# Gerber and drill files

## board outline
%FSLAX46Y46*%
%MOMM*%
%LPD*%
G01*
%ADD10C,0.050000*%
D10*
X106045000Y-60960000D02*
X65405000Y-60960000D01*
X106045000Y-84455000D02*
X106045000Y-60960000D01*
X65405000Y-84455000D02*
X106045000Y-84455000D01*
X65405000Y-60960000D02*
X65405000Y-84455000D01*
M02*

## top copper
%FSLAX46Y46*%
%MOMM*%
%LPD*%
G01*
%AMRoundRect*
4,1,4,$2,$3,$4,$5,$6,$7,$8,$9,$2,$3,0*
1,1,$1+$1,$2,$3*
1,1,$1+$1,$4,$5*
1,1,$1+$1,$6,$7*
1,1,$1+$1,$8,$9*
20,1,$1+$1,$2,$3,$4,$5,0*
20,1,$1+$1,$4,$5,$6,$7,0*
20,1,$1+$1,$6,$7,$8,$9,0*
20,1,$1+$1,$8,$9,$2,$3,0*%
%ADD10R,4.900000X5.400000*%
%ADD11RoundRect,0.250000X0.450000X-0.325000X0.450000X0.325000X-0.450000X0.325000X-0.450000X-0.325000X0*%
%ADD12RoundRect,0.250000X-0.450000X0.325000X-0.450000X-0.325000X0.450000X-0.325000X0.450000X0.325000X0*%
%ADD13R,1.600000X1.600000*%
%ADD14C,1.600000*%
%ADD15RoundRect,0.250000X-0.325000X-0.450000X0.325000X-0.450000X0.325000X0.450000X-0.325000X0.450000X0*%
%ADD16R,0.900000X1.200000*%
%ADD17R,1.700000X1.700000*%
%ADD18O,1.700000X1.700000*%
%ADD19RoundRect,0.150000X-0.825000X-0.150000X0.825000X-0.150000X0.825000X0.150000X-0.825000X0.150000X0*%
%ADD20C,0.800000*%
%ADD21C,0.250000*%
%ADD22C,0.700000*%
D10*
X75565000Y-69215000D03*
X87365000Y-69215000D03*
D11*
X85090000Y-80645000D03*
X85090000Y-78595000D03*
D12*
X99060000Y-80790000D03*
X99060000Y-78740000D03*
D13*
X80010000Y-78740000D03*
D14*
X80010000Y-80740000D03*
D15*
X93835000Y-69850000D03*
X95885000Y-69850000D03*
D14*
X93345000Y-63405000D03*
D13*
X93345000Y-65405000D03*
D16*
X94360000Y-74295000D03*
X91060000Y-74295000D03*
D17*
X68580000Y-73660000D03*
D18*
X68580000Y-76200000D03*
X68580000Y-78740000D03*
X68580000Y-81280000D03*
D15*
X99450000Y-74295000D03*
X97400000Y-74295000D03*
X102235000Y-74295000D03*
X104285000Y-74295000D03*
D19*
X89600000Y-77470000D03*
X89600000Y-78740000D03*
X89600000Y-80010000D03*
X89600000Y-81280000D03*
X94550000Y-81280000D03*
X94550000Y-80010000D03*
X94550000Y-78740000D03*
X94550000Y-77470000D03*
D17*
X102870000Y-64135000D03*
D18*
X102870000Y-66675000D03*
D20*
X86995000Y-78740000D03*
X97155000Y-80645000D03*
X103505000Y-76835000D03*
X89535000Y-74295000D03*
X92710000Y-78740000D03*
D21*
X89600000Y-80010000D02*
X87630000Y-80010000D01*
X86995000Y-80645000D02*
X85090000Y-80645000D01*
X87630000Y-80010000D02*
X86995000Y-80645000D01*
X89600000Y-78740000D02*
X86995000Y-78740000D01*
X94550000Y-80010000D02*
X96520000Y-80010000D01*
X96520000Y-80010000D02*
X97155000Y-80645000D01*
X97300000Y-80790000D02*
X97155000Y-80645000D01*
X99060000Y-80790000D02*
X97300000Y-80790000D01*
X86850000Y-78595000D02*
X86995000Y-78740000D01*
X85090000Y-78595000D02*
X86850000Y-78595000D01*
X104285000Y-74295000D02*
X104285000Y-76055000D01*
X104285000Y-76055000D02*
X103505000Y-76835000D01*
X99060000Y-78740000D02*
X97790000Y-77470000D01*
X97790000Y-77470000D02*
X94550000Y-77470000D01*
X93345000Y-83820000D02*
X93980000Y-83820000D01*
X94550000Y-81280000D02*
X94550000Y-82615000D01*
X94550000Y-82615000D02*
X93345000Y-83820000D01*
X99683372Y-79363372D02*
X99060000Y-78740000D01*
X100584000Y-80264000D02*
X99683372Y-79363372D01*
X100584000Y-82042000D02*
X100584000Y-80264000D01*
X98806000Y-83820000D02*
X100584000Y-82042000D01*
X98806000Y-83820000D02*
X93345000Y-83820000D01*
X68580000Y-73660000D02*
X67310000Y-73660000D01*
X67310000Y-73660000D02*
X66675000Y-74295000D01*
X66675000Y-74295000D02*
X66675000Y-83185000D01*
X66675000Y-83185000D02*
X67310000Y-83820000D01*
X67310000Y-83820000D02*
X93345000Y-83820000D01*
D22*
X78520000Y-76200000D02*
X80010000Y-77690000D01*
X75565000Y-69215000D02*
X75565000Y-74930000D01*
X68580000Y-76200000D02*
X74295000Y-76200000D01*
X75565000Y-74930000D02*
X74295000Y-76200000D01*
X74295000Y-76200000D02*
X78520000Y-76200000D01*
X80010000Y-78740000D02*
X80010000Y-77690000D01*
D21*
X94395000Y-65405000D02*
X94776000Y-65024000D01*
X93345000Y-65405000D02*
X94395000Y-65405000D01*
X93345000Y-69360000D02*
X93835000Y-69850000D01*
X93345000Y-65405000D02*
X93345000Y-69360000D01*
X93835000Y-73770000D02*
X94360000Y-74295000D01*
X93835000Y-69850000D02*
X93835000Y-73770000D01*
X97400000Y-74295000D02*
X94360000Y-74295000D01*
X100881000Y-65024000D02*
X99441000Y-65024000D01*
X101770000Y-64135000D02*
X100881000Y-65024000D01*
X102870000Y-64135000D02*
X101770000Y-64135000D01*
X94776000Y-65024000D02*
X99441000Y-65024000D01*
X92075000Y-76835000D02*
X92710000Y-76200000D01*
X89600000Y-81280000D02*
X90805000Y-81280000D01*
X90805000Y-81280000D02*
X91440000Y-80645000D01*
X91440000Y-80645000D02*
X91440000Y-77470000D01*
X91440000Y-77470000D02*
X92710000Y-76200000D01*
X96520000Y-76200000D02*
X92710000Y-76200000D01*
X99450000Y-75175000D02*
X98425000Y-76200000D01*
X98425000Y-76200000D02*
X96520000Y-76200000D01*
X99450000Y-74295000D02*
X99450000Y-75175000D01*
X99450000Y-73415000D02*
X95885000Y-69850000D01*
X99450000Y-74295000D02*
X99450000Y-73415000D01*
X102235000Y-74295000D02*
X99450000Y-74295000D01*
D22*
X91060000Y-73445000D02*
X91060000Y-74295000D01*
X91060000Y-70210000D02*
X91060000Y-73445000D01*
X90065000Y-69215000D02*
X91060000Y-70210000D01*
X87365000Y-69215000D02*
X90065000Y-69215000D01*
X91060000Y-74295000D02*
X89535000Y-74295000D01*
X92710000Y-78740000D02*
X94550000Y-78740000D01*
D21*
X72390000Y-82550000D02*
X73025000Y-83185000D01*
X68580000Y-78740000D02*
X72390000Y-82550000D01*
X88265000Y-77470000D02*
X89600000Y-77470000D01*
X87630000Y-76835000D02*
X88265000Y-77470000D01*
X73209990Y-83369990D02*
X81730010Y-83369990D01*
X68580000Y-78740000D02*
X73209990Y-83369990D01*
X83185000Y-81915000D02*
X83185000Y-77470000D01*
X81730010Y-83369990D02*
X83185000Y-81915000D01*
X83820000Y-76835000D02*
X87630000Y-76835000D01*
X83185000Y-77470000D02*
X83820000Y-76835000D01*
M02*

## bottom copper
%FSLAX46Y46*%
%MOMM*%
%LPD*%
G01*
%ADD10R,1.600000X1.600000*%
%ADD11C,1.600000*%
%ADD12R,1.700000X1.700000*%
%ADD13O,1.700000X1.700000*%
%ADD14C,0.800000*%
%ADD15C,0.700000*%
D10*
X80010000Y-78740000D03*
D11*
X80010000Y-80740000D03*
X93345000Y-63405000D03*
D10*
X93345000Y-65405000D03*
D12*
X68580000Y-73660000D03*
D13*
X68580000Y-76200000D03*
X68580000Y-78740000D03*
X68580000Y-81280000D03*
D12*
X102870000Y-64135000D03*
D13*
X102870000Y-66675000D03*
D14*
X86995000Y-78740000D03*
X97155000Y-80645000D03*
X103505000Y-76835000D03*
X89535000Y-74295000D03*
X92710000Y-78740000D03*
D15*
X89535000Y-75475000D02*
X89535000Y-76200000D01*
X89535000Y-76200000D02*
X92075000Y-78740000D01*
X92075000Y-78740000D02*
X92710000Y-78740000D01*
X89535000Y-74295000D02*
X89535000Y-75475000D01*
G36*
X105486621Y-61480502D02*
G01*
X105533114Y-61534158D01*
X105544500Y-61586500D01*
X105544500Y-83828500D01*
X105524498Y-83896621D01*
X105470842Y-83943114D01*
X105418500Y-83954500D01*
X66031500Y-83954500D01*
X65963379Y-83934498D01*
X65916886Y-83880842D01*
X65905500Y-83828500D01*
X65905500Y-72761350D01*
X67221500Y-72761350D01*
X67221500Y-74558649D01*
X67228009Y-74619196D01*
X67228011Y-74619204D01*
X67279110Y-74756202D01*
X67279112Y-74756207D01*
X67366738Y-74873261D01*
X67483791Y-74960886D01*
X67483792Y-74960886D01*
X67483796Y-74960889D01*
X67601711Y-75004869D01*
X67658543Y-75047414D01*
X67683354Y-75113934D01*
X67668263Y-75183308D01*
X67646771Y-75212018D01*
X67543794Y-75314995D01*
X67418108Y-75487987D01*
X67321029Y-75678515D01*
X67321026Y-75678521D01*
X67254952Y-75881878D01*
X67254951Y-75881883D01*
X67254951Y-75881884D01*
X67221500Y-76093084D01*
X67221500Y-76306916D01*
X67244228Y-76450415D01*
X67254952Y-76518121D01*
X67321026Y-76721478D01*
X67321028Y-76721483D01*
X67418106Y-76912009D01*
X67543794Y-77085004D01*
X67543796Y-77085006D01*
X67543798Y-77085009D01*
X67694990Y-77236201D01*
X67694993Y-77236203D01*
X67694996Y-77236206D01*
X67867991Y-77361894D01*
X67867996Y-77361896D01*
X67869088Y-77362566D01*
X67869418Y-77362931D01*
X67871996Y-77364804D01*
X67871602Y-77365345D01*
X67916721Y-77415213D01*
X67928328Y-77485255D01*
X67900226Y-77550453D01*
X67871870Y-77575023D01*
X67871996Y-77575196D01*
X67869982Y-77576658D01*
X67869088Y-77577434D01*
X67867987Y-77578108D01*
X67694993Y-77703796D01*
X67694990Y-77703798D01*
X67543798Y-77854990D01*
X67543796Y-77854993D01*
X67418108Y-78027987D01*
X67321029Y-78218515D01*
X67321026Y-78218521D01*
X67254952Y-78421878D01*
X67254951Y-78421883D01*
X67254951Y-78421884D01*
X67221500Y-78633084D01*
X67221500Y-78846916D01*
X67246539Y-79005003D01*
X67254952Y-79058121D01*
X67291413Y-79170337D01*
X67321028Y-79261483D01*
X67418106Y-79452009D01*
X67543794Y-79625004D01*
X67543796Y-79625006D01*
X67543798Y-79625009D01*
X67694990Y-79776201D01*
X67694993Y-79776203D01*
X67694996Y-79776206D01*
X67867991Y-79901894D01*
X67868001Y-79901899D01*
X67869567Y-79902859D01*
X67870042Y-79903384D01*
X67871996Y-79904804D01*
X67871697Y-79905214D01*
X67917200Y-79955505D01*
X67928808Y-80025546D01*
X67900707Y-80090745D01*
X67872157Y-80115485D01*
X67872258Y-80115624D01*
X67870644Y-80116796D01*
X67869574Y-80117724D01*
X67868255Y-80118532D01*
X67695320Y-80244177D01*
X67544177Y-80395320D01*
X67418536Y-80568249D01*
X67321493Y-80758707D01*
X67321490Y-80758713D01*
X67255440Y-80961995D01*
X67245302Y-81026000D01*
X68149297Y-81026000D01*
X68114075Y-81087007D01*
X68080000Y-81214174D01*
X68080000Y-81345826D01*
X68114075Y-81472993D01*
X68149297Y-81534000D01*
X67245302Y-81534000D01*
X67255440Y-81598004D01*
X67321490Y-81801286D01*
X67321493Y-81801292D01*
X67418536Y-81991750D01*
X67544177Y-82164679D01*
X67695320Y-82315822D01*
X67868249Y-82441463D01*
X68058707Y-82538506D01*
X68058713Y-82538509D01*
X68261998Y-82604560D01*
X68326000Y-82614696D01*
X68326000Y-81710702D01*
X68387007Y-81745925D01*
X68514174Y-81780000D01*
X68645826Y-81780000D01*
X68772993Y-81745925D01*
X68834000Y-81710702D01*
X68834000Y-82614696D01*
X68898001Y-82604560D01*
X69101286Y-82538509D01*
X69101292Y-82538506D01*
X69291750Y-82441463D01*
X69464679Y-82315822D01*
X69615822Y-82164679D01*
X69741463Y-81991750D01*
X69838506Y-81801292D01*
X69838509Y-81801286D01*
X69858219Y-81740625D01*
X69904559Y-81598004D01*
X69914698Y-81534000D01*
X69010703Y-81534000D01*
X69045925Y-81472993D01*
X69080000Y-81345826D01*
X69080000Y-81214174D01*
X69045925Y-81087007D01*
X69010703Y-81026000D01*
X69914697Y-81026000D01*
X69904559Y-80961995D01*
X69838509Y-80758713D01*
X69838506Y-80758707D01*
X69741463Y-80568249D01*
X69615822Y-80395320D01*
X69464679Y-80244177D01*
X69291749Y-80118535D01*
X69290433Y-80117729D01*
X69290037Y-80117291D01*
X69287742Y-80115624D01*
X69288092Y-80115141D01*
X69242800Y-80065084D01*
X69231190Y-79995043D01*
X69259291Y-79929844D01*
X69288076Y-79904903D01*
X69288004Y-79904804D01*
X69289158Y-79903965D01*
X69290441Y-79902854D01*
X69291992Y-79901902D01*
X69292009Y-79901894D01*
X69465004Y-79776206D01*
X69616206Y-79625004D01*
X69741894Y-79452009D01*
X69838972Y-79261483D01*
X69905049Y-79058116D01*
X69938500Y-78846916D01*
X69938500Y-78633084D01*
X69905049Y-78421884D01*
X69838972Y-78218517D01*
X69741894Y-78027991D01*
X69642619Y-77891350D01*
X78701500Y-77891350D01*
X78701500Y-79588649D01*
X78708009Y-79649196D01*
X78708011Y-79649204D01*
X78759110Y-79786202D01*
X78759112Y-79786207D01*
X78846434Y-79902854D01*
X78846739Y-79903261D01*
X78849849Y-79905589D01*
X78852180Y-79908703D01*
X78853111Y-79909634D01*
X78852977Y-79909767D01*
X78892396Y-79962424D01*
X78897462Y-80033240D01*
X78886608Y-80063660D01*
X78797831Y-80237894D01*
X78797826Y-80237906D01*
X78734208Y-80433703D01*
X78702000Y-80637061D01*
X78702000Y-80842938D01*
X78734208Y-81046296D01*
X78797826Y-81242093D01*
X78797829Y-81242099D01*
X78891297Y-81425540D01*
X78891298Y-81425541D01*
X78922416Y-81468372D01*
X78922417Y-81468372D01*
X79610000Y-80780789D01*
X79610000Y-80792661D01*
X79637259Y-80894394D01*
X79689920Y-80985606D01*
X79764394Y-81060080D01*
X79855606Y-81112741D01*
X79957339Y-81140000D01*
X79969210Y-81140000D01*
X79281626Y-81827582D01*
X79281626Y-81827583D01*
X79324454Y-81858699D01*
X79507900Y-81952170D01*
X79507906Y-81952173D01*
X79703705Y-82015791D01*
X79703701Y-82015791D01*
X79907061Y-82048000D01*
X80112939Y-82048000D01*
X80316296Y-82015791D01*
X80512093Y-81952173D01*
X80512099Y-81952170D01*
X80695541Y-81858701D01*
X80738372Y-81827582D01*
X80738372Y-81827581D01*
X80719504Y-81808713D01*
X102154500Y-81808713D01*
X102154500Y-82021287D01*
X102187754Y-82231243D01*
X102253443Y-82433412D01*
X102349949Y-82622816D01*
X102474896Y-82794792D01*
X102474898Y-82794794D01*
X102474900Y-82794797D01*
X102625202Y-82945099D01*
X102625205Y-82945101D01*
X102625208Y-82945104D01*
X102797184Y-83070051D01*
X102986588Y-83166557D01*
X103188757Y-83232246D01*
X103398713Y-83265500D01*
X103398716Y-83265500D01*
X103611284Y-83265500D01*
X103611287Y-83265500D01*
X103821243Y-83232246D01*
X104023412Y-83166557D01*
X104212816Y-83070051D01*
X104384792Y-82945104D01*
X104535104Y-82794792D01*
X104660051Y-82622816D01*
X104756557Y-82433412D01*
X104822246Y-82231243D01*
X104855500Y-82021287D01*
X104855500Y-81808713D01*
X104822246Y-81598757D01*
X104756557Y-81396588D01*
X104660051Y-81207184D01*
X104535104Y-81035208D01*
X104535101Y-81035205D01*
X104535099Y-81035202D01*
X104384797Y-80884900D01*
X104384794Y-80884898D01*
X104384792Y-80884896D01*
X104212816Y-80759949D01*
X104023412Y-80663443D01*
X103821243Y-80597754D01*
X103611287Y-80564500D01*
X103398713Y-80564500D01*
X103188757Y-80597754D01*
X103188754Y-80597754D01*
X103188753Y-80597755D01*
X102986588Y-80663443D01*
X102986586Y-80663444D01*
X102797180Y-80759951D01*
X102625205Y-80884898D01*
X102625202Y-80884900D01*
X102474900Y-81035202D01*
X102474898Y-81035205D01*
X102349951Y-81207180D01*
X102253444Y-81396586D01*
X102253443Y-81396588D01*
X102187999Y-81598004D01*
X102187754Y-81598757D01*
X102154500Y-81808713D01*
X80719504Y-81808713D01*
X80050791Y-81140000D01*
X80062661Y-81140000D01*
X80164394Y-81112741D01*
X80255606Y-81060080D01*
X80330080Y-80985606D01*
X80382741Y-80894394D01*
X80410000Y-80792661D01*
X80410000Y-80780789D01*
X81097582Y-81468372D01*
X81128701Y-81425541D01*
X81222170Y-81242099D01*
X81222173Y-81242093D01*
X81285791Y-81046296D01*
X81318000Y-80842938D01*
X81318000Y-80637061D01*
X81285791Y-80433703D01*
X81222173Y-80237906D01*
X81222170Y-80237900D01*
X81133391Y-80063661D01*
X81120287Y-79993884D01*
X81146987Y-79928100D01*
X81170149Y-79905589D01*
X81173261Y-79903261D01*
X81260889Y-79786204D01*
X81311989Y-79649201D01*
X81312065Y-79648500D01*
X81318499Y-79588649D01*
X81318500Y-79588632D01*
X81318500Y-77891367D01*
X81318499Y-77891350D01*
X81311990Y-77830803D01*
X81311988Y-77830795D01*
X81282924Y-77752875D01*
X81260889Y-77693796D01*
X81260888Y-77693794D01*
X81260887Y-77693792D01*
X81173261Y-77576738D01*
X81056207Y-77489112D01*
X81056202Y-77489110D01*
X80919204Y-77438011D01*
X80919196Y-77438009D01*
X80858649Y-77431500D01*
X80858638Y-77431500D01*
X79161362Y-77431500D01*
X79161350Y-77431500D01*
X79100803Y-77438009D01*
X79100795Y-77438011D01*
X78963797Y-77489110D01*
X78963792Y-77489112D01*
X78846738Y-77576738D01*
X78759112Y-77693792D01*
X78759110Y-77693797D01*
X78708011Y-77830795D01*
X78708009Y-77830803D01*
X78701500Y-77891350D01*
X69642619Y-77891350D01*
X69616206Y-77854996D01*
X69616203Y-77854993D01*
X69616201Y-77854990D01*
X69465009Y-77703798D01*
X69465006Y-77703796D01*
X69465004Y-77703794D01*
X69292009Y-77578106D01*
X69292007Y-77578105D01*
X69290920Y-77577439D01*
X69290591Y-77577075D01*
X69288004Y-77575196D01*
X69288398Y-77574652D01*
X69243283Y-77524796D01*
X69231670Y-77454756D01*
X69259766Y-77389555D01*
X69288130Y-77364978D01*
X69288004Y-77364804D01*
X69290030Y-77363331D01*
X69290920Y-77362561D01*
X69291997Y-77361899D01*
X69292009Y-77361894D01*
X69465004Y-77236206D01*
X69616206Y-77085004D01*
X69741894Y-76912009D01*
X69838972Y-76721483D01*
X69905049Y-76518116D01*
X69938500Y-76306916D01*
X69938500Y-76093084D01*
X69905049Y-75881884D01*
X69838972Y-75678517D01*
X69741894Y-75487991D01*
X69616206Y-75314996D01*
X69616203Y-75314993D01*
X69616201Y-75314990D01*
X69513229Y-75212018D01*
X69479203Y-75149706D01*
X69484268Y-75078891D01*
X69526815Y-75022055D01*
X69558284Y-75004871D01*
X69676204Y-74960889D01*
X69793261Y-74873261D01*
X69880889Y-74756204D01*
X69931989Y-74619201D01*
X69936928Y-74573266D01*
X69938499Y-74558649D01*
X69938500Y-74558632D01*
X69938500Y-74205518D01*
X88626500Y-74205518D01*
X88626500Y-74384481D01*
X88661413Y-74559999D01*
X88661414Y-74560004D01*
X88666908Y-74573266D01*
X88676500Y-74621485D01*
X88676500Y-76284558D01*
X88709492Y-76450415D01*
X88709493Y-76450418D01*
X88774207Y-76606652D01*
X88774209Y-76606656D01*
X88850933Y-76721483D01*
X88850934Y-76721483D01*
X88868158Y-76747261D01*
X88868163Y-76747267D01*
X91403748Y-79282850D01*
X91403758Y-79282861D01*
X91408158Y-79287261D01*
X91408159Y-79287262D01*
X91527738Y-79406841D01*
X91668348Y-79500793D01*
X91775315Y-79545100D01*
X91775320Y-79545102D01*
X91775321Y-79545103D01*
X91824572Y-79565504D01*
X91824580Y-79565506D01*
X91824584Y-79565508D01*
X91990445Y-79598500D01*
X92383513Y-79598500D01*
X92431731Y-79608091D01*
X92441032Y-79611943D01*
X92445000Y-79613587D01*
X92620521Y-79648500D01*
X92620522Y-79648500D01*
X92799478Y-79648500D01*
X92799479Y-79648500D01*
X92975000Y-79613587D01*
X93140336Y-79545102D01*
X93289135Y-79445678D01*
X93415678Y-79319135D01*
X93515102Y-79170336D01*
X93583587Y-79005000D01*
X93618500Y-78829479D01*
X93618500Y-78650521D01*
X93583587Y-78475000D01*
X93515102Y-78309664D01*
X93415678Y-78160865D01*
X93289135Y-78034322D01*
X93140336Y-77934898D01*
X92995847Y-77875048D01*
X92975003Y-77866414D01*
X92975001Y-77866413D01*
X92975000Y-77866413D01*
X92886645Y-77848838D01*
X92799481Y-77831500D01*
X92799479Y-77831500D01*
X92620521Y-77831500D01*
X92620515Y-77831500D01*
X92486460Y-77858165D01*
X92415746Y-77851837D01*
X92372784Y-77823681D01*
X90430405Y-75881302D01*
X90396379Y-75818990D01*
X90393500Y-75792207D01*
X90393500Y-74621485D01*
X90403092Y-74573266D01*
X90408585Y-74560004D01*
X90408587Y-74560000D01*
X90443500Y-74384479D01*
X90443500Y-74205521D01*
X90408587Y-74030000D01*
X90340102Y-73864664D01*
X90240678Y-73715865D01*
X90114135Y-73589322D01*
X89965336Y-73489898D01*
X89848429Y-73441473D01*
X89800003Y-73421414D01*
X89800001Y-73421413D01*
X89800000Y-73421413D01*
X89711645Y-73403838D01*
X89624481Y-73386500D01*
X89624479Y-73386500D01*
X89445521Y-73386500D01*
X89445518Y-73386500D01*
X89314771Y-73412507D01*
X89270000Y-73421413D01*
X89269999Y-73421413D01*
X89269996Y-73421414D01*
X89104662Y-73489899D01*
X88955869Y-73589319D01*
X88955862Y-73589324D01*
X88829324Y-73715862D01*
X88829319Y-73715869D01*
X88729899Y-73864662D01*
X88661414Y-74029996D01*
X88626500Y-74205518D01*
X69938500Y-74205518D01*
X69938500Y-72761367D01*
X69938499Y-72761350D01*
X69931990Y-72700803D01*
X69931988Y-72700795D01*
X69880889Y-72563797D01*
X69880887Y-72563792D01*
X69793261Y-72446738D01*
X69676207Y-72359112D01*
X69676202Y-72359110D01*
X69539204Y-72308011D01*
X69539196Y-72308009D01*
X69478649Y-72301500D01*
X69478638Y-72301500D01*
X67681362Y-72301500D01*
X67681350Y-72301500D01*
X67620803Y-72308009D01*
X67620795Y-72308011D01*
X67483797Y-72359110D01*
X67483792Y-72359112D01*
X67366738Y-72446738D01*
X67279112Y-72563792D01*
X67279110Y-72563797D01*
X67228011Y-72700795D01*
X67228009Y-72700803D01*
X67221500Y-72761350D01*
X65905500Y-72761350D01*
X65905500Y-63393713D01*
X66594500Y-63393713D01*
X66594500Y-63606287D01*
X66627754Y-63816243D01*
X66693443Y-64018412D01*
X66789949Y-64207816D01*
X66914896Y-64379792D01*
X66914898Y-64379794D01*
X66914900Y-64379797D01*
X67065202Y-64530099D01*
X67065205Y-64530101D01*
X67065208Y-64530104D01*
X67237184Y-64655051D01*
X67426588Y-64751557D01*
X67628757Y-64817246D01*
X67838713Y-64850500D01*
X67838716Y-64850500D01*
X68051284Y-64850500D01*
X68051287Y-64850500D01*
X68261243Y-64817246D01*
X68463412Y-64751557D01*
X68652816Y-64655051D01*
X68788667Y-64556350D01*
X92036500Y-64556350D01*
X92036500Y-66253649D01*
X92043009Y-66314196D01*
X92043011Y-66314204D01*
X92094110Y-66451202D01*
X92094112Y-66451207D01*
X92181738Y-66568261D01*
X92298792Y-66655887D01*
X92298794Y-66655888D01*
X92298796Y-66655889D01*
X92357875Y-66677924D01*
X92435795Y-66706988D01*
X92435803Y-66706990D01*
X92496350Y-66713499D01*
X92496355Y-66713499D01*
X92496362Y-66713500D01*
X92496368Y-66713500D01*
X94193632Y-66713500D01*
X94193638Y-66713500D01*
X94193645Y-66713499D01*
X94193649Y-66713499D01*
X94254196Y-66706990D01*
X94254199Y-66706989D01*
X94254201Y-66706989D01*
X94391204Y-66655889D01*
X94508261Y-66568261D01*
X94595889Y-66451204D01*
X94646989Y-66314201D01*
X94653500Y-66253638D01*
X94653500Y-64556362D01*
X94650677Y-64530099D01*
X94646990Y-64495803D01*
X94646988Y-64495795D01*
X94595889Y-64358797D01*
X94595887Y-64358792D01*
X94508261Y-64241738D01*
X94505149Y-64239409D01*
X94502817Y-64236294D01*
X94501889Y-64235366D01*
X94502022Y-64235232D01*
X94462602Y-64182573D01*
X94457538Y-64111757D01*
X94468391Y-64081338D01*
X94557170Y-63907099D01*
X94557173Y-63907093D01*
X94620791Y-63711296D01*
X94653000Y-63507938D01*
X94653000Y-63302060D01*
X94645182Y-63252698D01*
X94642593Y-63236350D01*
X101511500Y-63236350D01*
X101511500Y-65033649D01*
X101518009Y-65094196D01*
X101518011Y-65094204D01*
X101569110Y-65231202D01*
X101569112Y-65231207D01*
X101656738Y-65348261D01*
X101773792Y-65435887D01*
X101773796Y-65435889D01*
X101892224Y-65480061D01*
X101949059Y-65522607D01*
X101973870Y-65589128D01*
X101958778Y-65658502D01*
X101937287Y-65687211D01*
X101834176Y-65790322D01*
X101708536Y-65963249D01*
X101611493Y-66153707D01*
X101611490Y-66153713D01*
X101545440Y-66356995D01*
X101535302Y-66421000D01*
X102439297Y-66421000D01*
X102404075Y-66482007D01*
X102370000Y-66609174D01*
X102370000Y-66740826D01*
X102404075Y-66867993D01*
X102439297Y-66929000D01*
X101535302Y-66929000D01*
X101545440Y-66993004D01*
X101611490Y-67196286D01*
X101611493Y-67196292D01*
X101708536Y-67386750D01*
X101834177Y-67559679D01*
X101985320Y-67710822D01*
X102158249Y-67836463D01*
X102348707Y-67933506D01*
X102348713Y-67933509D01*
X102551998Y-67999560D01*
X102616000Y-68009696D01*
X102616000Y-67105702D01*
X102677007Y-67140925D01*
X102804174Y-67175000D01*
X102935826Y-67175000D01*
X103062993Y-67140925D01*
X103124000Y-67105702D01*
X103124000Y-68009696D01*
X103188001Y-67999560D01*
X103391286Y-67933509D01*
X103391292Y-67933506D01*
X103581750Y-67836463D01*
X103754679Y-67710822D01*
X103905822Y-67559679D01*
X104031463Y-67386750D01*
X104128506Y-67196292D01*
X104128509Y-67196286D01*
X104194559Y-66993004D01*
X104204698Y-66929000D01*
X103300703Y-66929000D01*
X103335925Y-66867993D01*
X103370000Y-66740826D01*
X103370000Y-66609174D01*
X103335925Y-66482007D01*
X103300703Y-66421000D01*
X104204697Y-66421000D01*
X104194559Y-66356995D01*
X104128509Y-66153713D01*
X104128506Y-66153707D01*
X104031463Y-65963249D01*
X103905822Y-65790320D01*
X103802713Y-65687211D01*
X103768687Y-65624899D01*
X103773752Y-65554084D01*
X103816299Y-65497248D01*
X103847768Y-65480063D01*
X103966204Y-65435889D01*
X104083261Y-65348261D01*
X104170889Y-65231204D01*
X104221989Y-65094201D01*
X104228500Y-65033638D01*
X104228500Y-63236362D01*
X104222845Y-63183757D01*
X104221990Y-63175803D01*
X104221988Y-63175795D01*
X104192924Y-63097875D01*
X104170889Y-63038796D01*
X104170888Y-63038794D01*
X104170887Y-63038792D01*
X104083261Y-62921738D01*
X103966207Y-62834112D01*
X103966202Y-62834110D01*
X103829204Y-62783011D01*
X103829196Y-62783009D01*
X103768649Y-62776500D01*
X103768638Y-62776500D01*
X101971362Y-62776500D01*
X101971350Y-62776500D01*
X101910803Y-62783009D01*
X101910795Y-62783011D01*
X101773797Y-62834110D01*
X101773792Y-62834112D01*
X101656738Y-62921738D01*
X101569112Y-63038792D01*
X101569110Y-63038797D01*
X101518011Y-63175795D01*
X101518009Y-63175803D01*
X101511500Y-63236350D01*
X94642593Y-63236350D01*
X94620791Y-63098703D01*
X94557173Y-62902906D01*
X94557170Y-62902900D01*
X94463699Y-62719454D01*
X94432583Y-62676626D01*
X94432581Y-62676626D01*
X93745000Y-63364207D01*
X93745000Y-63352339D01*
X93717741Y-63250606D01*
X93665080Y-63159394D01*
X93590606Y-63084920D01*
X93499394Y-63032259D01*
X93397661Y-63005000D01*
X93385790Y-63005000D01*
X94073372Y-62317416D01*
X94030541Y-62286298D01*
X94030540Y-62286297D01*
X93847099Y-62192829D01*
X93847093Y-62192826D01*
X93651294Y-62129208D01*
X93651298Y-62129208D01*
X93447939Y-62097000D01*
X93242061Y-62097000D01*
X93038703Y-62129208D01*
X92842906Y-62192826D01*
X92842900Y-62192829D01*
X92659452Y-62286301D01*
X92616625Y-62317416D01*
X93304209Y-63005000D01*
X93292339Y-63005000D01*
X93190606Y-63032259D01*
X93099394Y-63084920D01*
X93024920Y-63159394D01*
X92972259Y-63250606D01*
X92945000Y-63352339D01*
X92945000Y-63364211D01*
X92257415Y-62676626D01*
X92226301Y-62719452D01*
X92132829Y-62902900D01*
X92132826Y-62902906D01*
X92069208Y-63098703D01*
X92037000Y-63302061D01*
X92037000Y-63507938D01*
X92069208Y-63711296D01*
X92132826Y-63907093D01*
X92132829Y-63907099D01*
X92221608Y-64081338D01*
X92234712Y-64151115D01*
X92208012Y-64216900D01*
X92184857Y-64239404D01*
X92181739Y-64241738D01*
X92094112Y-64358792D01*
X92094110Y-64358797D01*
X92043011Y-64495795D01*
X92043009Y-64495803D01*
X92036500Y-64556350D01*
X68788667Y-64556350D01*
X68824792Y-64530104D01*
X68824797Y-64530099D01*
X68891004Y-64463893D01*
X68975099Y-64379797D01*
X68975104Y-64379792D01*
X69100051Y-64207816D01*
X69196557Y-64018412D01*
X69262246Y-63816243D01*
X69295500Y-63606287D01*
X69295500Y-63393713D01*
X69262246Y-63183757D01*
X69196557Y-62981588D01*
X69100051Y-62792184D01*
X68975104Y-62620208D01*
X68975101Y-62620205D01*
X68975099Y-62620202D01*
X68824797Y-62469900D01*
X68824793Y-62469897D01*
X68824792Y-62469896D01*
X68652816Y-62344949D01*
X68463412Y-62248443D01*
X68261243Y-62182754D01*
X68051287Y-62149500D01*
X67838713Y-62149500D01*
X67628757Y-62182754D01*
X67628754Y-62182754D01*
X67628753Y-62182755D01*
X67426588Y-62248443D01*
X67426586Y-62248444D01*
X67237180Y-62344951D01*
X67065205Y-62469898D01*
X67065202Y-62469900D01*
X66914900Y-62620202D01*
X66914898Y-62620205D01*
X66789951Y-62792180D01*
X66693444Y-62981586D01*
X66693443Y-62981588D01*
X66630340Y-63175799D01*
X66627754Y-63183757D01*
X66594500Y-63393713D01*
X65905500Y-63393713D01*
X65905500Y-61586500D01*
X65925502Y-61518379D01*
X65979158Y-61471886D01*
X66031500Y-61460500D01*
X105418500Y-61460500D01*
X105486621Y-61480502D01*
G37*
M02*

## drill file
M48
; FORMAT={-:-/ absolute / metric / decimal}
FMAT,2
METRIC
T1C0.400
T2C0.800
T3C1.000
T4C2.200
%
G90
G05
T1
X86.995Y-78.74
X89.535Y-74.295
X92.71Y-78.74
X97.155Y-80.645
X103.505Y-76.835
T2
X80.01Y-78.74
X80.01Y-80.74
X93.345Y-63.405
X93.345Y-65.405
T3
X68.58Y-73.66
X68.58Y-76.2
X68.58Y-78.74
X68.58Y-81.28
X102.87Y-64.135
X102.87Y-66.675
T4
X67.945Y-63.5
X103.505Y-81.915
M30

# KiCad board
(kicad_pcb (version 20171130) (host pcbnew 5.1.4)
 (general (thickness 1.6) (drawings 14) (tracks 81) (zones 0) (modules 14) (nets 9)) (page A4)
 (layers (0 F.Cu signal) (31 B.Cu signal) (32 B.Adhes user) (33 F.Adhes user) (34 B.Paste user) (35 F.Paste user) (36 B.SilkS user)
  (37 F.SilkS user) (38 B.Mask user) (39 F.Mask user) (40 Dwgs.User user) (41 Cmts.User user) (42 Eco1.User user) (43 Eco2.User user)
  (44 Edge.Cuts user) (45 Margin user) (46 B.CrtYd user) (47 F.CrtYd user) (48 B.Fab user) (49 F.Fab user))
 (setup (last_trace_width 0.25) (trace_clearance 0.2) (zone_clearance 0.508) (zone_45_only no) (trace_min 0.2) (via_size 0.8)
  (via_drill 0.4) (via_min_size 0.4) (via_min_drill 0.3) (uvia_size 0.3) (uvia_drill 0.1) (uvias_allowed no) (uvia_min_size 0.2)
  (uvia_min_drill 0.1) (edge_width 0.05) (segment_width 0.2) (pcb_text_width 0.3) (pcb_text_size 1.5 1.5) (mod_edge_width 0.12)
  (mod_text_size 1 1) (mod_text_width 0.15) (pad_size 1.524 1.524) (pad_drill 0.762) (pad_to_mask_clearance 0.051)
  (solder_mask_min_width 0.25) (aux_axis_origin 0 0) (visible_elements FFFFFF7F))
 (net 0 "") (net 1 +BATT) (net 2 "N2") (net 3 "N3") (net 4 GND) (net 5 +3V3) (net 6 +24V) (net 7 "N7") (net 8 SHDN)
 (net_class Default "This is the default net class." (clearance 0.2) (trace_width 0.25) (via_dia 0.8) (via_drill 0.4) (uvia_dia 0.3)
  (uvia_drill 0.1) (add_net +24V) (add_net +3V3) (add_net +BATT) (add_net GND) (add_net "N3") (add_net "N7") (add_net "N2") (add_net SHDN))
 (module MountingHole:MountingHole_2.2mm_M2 (layer F.Cu) (at 103.505 81.915)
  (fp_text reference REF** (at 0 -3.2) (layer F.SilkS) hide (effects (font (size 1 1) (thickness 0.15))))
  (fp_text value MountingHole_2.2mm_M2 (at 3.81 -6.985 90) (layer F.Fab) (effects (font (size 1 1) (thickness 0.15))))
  (pad 1 np_thru_hole circle (at 0 0) (size 2.2 2.2) (drill 2.2) (layers *.Cu *.Mask)))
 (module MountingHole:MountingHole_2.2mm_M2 (layer F.Cu) (at 67.945 63.5)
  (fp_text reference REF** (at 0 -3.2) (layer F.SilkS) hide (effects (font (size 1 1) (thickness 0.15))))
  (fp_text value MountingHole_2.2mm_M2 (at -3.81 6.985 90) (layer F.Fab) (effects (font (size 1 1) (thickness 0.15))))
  (pad 1 np_thru_hole circle (at 0 0) (size 2.2 2.2) (drill 2.2) (layers *.Cu *.Mask)))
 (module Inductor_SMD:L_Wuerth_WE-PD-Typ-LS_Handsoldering (layer F.Cu) (at 81.465 69.215)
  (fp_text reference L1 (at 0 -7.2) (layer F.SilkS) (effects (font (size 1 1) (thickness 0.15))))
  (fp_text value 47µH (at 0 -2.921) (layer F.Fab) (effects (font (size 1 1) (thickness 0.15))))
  (pad 1 smd rect (at -5.9 0) (size 4.9 5.4) (layers F.Cu F.Paste F.Mask) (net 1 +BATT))
  (pad 2 smd rect (at 5.9 0) (size 4.9 5.4) (layers F.Cu F.Paste F.Mask) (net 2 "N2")))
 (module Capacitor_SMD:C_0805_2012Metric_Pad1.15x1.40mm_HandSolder (layer F.Cu) (at 85.09 79.62 90)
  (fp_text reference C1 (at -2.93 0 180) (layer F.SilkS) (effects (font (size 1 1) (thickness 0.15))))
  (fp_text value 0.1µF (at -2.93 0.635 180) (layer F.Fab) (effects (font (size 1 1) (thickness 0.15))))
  (pad 1 smd roundrect (at -1.025 0 90) (size 1.15 1.4) (layers F.Cu F.Paste F.Mask) (roundrect_rratio 0.217391) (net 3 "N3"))
  (pad 2 smd roundrect (at 1.025 0 90) (size 1.15 1.4) (layers F.Cu F.Paste F.Mask) (roundrect_rratio 0.217391) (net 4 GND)))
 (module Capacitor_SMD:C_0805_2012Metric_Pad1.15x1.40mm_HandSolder (layer F.Cu) (at 99.06 79.765 270)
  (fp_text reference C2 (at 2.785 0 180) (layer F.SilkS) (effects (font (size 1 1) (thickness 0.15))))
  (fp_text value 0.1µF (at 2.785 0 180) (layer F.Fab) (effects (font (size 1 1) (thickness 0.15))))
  (pad 2 smd roundrect (at 1.025 0 270) (size 1.15 1.4) (layers F.Cu F.Paste F.Mask) (roundrect_rratio 0.217391) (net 4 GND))
  (pad 1 smd roundrect (at -1.025 0 270) (size 1.15 1.4) (layers F.Cu F.Paste F.Mask) (roundrect_rratio 0.217391) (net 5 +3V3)))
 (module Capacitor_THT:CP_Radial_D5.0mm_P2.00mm (layer F.Cu) (at 80.01 78.74 270)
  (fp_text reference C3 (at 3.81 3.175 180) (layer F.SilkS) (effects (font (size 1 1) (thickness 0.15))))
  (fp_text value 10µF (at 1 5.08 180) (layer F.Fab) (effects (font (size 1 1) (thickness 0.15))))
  (pad 1 thru_hole rect (at 0 0 270) (size 1.6 1.6) (drill 0.8) (layers *.Cu *.Mask) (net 1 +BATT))
  (pad 2 thru_hole circle (at 2 0 270) (size 1.6 1.6) (drill 0.8) (layers *.Cu *.Mask) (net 4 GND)))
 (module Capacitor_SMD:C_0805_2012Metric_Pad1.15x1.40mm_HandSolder (layer F.Cu) (at 94.86 69.85)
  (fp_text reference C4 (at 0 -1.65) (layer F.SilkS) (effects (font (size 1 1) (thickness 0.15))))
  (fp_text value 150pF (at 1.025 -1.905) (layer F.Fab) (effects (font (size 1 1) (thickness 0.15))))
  (pad 1 smd roundrect (at -1.025 0) (size 1.15 1.4) (layers F.Cu F.Paste F.Mask) (roundrect_rratio 0.217391) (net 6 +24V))
  (pad 2 smd roundrect (at 1.025 0) (size 1.15 1.4) (layers F.Cu F.Paste F.Mask) (roundrect_rratio 0.217391) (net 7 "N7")))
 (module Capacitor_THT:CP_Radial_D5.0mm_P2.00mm (layer F.Cu) (at 93.345 65.405 90)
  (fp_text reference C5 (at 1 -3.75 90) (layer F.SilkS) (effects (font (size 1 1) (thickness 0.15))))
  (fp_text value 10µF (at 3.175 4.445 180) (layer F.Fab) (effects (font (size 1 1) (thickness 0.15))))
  (pad 2 thru_hole circle (at 2 0 90) (size 1.6 1.6) (drill 0.8) (layers *.Cu *.Mask) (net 4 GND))
  (pad 1 thru_hole rect (at 0 0 90) (size 1.6 1.6) (drill 0.8) (layers *.Cu *.Mask) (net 6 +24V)))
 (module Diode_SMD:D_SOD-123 (layer F.Cu) (at 92.71 74.295 180)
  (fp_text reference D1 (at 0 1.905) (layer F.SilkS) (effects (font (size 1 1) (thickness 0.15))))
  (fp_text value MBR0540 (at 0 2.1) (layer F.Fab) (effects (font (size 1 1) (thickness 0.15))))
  (pad 1 smd rect (at -1.65 0 180) (size 0.9 1.2) (layers F.Cu F.Paste F.Mask) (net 6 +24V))
  (pad 2 smd rect (at 1.65 0 180) (size 0.9 1.2) (layers F.Cu F.Paste F.Mask) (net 2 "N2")))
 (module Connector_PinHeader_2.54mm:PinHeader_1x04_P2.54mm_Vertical (layer F.Cu) (at 68.58 73.66)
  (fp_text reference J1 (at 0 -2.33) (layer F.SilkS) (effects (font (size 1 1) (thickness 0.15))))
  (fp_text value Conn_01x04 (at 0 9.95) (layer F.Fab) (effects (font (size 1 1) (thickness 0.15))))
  (pad 1 thru_hole rect (at 0 0) (size 1.7 1.7) (drill 1) (layers *.Cu *.Mask) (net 5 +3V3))
  (pad 2 thru_hole oval (at 0 2.54) (size 1.7 1.7) (drill 1) (layers *.Cu *.Mask) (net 1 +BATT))
  (pad 3 thru_hole oval (at 0 5.08) (size 1.7 1.7) (drill 1) (layers *.Cu *.Mask) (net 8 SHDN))
  (pad 4 thru_hole oval (at 0 7.62) (size 1.7 1.7) (drill 1) (layers *.Cu *.Mask) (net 4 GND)))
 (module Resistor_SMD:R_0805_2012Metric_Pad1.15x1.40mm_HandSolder (layer F.Cu) (at 98.425 74.295)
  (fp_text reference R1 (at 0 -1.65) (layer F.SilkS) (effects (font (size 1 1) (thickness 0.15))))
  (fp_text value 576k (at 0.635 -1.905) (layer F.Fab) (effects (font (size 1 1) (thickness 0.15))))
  (pad 2 smd roundrect (at 1.025 0) (size 1.15 1.4) (layers F.Cu F.Paste F.Mask) (roundrect_rratio 0.217391) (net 7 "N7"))
  (pad 1 smd roundrect (at -1.025 0) (size 1.15 1.4) (layers F.Cu F.Paste F.Mask) (roundrect_rratio 0.217391) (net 6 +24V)))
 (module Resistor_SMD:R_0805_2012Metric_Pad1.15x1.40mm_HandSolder (layer F.Cu) (at 103.26 74.295)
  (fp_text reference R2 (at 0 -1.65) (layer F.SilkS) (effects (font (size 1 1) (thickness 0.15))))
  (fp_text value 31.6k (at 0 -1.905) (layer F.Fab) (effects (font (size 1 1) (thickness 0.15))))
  (pad 1 smd roundrect (at -1.025 0) (size 1.15 1.4) (layers F.Cu F.Paste F.Mask) (roundrect_rratio 0.217391) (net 7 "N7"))
  (pad 2 smd roundrect (at 1.025 0) (size 1.15 1.4) (layers F.Cu F.Paste F.Mask) (roundrect_rratio 0.217391) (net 4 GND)))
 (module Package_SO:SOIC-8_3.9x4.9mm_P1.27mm (layer F.Cu) (at 92.075 79.375)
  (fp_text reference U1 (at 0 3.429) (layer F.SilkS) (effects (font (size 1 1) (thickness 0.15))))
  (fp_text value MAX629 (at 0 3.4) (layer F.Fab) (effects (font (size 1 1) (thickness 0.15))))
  (pad 1 smd roundrect (at -2.475 -1.905) (size 1.95 0.6) (layers F.Cu F.Paste F.Mask) (roundrect_rratio 0.25) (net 8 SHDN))
  (pad 2 smd roundrect (at -2.475 -0.635) (size 1.95 0.6) (layers F.Cu F.Paste F.Mask) (roundrect_rratio 0.25) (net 4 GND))
  (pad 3 smd roundrect (at -2.475 0.635) (size 1.95 0.6) (layers F.Cu F.Paste F.Mask) (roundrect_rratio 0.25) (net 3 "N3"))
  (pad 4 smd roundrect (at -2.475 1.905) (size 1.95 0.6) (layers F.Cu F.Paste F.Mask) (roundrect_rratio 0.25) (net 7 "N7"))
  (pad 5 smd roundrect (at 2.475 1.905) (size 1.95 0.6) (layers F.Cu F.Paste F.Mask) (roundrect_rratio 0.25) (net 5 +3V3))
  (pad 6 smd roundrect (at 2.475 0.635) (size 1.95 0.6) (layers F.Cu F.Paste F.Mask) (roundrect_rratio 0.25) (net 4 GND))
  (pad 7 smd roundrect (at 2.475 -0.635) (size 1.95 0.6) (layers F.Cu F.Paste F.Mask) (roundrect_rratio 0.25) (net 2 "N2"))
  (pad 8 smd roundrect (at 2.475 -1.905) (size 1.95 0.6) (layers F.Cu F.Paste F.Mask) (roundrect_rratio 0.25) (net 5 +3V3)))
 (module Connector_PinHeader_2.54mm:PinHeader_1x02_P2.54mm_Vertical (layer F.Cu) (at 102.87 64.135)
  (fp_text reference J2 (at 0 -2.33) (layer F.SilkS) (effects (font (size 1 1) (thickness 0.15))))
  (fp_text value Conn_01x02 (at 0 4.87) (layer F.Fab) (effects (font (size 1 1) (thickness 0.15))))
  (pad 1 thru_hole rect (at 0 0) (size 1.7 1.7) (drill 1) (layers *.Cu *.Mask) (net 6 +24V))
  (pad 2 thru_hole oval (at 0 2.54) (size 1.7 1.7) (drill 1) (layers *.Cu *.Mask) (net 4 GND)))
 (gr_line (start 106.045 60.96) (end 65.405 60.96) (layer Edge.Cuts) (width 0.05))
 (gr_line (start 106.045 84.455) (end 106.045 60.96) (layer Edge.Cuts) (width 0.05))
 (gr_line (start 65.405 84.455) (end 106.045 84.455) (layer Edge.Cuts) (width 0.05))
 (gr_line (start 65.405 60.96) (end 65.405 84.455) (layer Edge.Cuts) (width 0.05))
 (segment (start 89.6 80.01) (end 87.63 80.01) (width 0.25) (layer F.Cu) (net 3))
 (segment (start 86.995 80.645) (end 85.09 80.645) (width 0.25) (layer F.Cu) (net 3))
 (segment (start 87.63 80.01) (end 86.995 80.645) (width 0.25) (layer F.Cu) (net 3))
 (via (at 86.995 78.74) (size 0.8) (drill 0.4) (layers F.Cu B.Cu) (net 4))
 (segment (start 89.6 78.74) (end 86.995 78.74) (width 0.25) (layer F.Cu) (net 4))
 (via (at 97.155 80.645) (size 0.8) (drill 0.4) (layers F.Cu B.Cu) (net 4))
 (segment (start 94.55 80.01) (end 96.52 80.01) (width 0.25) (layer F.Cu) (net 4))
 (segment (start 96.52 80.01) (end 97.155 80.645) (width 0.25) (layer F.Cu) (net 4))
 (segment (start 97.3 80.79) (end 97.155 80.645) (width 0.25) (layer F.Cu) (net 4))
 (segment (start 99.06 80.79) (end 97.3 80.79) (width 0.25) (layer F.Cu) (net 4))
 (segment (start 86.85 78.595) (end 86.995 78.74) (width 0.25) (layer F.Cu) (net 4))
 (segment (start 85.09 78.595) (end 86.85 78.595) (width 0.25) (layer F.Cu) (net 4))
 (segment (start 104.285 74.295) (end 104.285 76.055) (width 0.25) (layer F.Cu) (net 4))
 (via (at 103.505 76.835) (size 0.8) (drill 0.4) (layers F.Cu B.Cu) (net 4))
 (segment (start 104.285 76.055) (end 103.505 76.835) (width 0.25) (layer F.Cu) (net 4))
 (segment (start 99.06 78.74) (end 97.79 77.47) (width 0.25) (layer F.Cu) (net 5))
 (segment (start 97.79 77.47) (end 94.55 77.47) (width 0.25) (layer F.Cu) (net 5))
 (segment (start 93.345 83.82) (end 93.98 83.82) (width 0.25) (layer F.Cu) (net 5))
 (segment (start 94.55 81.28) (end 94.55 82.615) (width 0.25) (layer F.Cu) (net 5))
 (segment (start 94.55 82.615) (end 93.345 83.82) (width 0.25) (layer F.Cu) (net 5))
 (segment (start 99.683372 79.363372) (end 99.06 78.74) (width 0.25) (layer F.Cu) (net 5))
 (segment (start 100.584 80.264) (end 99.683372 79.363372) (width 0.25) (layer F.Cu) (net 5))
 (segment (start 100.584 82.042) (end 100.584 80.264) (width 0.25) (layer F.Cu) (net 5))
 (segment (start 98.806 83.82) (end 100.584 82.042) (width 0.25) (layer F.Cu) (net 5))
 (segment (start 98.806 83.82) (end 93.345 83.82) (width 0.25) (layer F.Cu) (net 5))
 (segment (start 68.58 73.66) (end 67.31 73.66) (width 0.25) (layer F.Cu) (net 5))
 (segment (start 67.31 73.66) (end 66.675 74.295) (width 0.25) (layer F.Cu) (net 5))
 (segment (start 66.675 74.295) (end 66.675 83.185) (width 0.25) (layer F.Cu) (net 5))
 (segment (start 66.675 83.185) (end 67.31 83.82) (width 0.25) (layer F.Cu) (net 5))
 (segment (start 67.31 83.82) (end 93.345 83.82) (width 0.25) (layer F.Cu) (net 5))
 (segment (start 78.52 76.2) (end 80.01 77.69) (width 0.7) (layer F.Cu) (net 1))
 (segment (start 75.565 69.215) (end 75.565 74.93) (width 0.7) (layer F.Cu) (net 1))
 (segment (start 68.58 76.2) (end 74.295 76.2) (width 0.7) (layer F.Cu) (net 1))
 (segment (start 75.565 74.93) (end 74.295 76.2) (width 0.7) (layer F.Cu) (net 1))
 (segment (start 74.295 76.2) (end 78.52 76.2) (width 0.7) (layer F.Cu) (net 1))
 (segment (start 80.01 78.74) (end 80.01 77.69) (width 0.7) (layer F.Cu) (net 1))
 (segment (start 94.395 65.405) (end 94.776 65.024) (width 0.25) (layer F.Cu) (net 6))
 (segment (start 93.345 65.405) (end 94.395 65.405) (width 0.25) (layer F.Cu) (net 6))
 (segment (start 93.345 69.36) (end 93.835 69.85) (width 0.25) (layer F.Cu) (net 6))
 (segment (start 93.345 65.405) (end 93.345 69.36) (width 0.25) (layer F.Cu) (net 6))
 (segment (start 93.835 73.77) (end 94.36 74.295) (width 0.25) (layer F.Cu) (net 6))
 (segment (start 93.835 69.85) (end 93.835 73.77) (width 0.25) (layer F.Cu) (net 6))
 (segment (start 97.4 74.295) (end 94.36 74.295) (width 0.25) (layer F.Cu) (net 6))
 (segment (start 100.881 65.024) (end 99.441 65.024) (width 0.25) (layer F.Cu) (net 6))
 (segment (start 101.77 64.135) (end 100.881 65.024) (width 0.25) (layer F.Cu) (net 6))
 (segment (start 102.87 64.135) (end 101.77 64.135) (width 0.25) (layer F.Cu) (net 6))
 (segment (start 94.776 65.024) (end 99.441 65.024) (width 0.25) (layer F.Cu) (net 6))
 (segment (start 92.075 76.835) (end 92.71 76.2) (width 0.25) (layer F.Cu) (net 7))
 (segment (start 89.6 81.28) (end 90.805 81.28) (width 0.25) (layer F.Cu) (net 7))
 (segment (start 90.805 81.28) (end 91.44 80.645) (width 0.25) (layer F.Cu) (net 7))
 (segment (start 91.44 80.645) (end 91.44 77.47) (width 0.25) (layer F.Cu) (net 7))
 (segment (start 91.44 77.47) (end 92.71 76.2) (width 0.25) (layer F.Cu) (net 7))
 (segment (start 96.52 76.2) (end 92.71 76.2) (width 0.25) (layer F.Cu) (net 7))
 (segment (start 99.45 75.175) (end 98.425 76.2) (width 0.25) (layer F.Cu) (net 7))
 (segment (start 98.425 76.2) (end 96.52 76.2) (width 0.25) (layer F.Cu) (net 7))
 (segment (start 99.45 74.295) (end 99.45 75.175) (width 0.25) (layer F.Cu) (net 7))
 (segment (start 99.45 73.415) (end 95.885 69.85) (width 0.25) (layer F.Cu) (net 7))
 (segment (start 99.45 74.295) (end 99.45 73.415) (width 0.25) (layer F.Cu) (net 7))
 (segment (start 102.235 74.295) (end 99.45 74.295) (width 0.25) (layer F.Cu) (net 7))
 (segment (start 91.06 73.445) (end 91.06 74.295) (width 0.7) (layer F.Cu) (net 2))
 (segment (start 91.06 70.21) (end 91.06 73.445) (width 0.7) (layer F.Cu) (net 2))
 (segment (start 90.065 69.215) (end 91.06 70.21) (width 0.7) (layer F.Cu) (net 2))
 (segment (start 87.365 69.215) (end 90.065 69.215) (width 0.7) (layer F.Cu) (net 2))
 (via (at 89.535 74.295) (size 0.8) (drill 0.4) (layers F.Cu B.Cu) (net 2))
 (segment (start 91.06 74.295) (end 89.535 74.295) (width 0.7) (layer F.Cu) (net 2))
 (segment (start 89.535 75.475) (end 89.535 76.2) (width 0.7) (layer B.Cu) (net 2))
 (segment (start 89.535 76.2) (end 92.075 78.74) (width 0.7) (layer B.Cu) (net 2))
 (via (at 92.71 78.74) (size 0.8) (drill 0.4) (layers F.Cu B.Cu) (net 2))
 (segment (start 92.075 78.74) (end 92.71 78.74) (width 0.7) (layer B.Cu) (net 2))
 (segment (start 92.71 78.74) (end 94.55 78.74) (width 0.7) (layer F.Cu) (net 2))
 (segment (start 89.535 74.295) (end 89.535 75.475) (width 0.7) (layer B.Cu) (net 2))
 (segment (start 72.39 82.55) (end 73.025 83.185) (width 0.25) (layer F.Cu) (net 8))
 (segment (start 68.58 78.74) (end 72.39 82.55) (width 0.25) (layer F.Cu) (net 8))
 (segment (start 88.265 77.47) (end 89.6 77.47) (width 0.25) (layer F.Cu) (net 8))
 (segment (start 87.63 76.835) (end 88.265 77.47) (width 0.25) (layer F.Cu) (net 8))
 (segment (start 73.20999 83.36999) (end 81.73001 83.36999) (width 0.25) (layer F.Cu) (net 8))
 (segment (start 68.58 78.74) (end 73.20999 83.36999) (width 0.25) (layer F.Cu) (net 8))
 (segment (start 83.185 81.915) (end 83.185 77.47) (width 0.25) (layer F.Cu) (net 8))
 (segment (start 81.73001 83.36999) (end 83.185 81.915) (width 0.25) (layer F.Cu) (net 8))
 (segment (start 83.82 76.835) (end 87.63 76.835) (width 0.25) (layer F.Cu) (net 8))
 (segment (start 83.185 77.47) (end 83.82 76.835) (width 0.25) (layer F.Cu) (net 8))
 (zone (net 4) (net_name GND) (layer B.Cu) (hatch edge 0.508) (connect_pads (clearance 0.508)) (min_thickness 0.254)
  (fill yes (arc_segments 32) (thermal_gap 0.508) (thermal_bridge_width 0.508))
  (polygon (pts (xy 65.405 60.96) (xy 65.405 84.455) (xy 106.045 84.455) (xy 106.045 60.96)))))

